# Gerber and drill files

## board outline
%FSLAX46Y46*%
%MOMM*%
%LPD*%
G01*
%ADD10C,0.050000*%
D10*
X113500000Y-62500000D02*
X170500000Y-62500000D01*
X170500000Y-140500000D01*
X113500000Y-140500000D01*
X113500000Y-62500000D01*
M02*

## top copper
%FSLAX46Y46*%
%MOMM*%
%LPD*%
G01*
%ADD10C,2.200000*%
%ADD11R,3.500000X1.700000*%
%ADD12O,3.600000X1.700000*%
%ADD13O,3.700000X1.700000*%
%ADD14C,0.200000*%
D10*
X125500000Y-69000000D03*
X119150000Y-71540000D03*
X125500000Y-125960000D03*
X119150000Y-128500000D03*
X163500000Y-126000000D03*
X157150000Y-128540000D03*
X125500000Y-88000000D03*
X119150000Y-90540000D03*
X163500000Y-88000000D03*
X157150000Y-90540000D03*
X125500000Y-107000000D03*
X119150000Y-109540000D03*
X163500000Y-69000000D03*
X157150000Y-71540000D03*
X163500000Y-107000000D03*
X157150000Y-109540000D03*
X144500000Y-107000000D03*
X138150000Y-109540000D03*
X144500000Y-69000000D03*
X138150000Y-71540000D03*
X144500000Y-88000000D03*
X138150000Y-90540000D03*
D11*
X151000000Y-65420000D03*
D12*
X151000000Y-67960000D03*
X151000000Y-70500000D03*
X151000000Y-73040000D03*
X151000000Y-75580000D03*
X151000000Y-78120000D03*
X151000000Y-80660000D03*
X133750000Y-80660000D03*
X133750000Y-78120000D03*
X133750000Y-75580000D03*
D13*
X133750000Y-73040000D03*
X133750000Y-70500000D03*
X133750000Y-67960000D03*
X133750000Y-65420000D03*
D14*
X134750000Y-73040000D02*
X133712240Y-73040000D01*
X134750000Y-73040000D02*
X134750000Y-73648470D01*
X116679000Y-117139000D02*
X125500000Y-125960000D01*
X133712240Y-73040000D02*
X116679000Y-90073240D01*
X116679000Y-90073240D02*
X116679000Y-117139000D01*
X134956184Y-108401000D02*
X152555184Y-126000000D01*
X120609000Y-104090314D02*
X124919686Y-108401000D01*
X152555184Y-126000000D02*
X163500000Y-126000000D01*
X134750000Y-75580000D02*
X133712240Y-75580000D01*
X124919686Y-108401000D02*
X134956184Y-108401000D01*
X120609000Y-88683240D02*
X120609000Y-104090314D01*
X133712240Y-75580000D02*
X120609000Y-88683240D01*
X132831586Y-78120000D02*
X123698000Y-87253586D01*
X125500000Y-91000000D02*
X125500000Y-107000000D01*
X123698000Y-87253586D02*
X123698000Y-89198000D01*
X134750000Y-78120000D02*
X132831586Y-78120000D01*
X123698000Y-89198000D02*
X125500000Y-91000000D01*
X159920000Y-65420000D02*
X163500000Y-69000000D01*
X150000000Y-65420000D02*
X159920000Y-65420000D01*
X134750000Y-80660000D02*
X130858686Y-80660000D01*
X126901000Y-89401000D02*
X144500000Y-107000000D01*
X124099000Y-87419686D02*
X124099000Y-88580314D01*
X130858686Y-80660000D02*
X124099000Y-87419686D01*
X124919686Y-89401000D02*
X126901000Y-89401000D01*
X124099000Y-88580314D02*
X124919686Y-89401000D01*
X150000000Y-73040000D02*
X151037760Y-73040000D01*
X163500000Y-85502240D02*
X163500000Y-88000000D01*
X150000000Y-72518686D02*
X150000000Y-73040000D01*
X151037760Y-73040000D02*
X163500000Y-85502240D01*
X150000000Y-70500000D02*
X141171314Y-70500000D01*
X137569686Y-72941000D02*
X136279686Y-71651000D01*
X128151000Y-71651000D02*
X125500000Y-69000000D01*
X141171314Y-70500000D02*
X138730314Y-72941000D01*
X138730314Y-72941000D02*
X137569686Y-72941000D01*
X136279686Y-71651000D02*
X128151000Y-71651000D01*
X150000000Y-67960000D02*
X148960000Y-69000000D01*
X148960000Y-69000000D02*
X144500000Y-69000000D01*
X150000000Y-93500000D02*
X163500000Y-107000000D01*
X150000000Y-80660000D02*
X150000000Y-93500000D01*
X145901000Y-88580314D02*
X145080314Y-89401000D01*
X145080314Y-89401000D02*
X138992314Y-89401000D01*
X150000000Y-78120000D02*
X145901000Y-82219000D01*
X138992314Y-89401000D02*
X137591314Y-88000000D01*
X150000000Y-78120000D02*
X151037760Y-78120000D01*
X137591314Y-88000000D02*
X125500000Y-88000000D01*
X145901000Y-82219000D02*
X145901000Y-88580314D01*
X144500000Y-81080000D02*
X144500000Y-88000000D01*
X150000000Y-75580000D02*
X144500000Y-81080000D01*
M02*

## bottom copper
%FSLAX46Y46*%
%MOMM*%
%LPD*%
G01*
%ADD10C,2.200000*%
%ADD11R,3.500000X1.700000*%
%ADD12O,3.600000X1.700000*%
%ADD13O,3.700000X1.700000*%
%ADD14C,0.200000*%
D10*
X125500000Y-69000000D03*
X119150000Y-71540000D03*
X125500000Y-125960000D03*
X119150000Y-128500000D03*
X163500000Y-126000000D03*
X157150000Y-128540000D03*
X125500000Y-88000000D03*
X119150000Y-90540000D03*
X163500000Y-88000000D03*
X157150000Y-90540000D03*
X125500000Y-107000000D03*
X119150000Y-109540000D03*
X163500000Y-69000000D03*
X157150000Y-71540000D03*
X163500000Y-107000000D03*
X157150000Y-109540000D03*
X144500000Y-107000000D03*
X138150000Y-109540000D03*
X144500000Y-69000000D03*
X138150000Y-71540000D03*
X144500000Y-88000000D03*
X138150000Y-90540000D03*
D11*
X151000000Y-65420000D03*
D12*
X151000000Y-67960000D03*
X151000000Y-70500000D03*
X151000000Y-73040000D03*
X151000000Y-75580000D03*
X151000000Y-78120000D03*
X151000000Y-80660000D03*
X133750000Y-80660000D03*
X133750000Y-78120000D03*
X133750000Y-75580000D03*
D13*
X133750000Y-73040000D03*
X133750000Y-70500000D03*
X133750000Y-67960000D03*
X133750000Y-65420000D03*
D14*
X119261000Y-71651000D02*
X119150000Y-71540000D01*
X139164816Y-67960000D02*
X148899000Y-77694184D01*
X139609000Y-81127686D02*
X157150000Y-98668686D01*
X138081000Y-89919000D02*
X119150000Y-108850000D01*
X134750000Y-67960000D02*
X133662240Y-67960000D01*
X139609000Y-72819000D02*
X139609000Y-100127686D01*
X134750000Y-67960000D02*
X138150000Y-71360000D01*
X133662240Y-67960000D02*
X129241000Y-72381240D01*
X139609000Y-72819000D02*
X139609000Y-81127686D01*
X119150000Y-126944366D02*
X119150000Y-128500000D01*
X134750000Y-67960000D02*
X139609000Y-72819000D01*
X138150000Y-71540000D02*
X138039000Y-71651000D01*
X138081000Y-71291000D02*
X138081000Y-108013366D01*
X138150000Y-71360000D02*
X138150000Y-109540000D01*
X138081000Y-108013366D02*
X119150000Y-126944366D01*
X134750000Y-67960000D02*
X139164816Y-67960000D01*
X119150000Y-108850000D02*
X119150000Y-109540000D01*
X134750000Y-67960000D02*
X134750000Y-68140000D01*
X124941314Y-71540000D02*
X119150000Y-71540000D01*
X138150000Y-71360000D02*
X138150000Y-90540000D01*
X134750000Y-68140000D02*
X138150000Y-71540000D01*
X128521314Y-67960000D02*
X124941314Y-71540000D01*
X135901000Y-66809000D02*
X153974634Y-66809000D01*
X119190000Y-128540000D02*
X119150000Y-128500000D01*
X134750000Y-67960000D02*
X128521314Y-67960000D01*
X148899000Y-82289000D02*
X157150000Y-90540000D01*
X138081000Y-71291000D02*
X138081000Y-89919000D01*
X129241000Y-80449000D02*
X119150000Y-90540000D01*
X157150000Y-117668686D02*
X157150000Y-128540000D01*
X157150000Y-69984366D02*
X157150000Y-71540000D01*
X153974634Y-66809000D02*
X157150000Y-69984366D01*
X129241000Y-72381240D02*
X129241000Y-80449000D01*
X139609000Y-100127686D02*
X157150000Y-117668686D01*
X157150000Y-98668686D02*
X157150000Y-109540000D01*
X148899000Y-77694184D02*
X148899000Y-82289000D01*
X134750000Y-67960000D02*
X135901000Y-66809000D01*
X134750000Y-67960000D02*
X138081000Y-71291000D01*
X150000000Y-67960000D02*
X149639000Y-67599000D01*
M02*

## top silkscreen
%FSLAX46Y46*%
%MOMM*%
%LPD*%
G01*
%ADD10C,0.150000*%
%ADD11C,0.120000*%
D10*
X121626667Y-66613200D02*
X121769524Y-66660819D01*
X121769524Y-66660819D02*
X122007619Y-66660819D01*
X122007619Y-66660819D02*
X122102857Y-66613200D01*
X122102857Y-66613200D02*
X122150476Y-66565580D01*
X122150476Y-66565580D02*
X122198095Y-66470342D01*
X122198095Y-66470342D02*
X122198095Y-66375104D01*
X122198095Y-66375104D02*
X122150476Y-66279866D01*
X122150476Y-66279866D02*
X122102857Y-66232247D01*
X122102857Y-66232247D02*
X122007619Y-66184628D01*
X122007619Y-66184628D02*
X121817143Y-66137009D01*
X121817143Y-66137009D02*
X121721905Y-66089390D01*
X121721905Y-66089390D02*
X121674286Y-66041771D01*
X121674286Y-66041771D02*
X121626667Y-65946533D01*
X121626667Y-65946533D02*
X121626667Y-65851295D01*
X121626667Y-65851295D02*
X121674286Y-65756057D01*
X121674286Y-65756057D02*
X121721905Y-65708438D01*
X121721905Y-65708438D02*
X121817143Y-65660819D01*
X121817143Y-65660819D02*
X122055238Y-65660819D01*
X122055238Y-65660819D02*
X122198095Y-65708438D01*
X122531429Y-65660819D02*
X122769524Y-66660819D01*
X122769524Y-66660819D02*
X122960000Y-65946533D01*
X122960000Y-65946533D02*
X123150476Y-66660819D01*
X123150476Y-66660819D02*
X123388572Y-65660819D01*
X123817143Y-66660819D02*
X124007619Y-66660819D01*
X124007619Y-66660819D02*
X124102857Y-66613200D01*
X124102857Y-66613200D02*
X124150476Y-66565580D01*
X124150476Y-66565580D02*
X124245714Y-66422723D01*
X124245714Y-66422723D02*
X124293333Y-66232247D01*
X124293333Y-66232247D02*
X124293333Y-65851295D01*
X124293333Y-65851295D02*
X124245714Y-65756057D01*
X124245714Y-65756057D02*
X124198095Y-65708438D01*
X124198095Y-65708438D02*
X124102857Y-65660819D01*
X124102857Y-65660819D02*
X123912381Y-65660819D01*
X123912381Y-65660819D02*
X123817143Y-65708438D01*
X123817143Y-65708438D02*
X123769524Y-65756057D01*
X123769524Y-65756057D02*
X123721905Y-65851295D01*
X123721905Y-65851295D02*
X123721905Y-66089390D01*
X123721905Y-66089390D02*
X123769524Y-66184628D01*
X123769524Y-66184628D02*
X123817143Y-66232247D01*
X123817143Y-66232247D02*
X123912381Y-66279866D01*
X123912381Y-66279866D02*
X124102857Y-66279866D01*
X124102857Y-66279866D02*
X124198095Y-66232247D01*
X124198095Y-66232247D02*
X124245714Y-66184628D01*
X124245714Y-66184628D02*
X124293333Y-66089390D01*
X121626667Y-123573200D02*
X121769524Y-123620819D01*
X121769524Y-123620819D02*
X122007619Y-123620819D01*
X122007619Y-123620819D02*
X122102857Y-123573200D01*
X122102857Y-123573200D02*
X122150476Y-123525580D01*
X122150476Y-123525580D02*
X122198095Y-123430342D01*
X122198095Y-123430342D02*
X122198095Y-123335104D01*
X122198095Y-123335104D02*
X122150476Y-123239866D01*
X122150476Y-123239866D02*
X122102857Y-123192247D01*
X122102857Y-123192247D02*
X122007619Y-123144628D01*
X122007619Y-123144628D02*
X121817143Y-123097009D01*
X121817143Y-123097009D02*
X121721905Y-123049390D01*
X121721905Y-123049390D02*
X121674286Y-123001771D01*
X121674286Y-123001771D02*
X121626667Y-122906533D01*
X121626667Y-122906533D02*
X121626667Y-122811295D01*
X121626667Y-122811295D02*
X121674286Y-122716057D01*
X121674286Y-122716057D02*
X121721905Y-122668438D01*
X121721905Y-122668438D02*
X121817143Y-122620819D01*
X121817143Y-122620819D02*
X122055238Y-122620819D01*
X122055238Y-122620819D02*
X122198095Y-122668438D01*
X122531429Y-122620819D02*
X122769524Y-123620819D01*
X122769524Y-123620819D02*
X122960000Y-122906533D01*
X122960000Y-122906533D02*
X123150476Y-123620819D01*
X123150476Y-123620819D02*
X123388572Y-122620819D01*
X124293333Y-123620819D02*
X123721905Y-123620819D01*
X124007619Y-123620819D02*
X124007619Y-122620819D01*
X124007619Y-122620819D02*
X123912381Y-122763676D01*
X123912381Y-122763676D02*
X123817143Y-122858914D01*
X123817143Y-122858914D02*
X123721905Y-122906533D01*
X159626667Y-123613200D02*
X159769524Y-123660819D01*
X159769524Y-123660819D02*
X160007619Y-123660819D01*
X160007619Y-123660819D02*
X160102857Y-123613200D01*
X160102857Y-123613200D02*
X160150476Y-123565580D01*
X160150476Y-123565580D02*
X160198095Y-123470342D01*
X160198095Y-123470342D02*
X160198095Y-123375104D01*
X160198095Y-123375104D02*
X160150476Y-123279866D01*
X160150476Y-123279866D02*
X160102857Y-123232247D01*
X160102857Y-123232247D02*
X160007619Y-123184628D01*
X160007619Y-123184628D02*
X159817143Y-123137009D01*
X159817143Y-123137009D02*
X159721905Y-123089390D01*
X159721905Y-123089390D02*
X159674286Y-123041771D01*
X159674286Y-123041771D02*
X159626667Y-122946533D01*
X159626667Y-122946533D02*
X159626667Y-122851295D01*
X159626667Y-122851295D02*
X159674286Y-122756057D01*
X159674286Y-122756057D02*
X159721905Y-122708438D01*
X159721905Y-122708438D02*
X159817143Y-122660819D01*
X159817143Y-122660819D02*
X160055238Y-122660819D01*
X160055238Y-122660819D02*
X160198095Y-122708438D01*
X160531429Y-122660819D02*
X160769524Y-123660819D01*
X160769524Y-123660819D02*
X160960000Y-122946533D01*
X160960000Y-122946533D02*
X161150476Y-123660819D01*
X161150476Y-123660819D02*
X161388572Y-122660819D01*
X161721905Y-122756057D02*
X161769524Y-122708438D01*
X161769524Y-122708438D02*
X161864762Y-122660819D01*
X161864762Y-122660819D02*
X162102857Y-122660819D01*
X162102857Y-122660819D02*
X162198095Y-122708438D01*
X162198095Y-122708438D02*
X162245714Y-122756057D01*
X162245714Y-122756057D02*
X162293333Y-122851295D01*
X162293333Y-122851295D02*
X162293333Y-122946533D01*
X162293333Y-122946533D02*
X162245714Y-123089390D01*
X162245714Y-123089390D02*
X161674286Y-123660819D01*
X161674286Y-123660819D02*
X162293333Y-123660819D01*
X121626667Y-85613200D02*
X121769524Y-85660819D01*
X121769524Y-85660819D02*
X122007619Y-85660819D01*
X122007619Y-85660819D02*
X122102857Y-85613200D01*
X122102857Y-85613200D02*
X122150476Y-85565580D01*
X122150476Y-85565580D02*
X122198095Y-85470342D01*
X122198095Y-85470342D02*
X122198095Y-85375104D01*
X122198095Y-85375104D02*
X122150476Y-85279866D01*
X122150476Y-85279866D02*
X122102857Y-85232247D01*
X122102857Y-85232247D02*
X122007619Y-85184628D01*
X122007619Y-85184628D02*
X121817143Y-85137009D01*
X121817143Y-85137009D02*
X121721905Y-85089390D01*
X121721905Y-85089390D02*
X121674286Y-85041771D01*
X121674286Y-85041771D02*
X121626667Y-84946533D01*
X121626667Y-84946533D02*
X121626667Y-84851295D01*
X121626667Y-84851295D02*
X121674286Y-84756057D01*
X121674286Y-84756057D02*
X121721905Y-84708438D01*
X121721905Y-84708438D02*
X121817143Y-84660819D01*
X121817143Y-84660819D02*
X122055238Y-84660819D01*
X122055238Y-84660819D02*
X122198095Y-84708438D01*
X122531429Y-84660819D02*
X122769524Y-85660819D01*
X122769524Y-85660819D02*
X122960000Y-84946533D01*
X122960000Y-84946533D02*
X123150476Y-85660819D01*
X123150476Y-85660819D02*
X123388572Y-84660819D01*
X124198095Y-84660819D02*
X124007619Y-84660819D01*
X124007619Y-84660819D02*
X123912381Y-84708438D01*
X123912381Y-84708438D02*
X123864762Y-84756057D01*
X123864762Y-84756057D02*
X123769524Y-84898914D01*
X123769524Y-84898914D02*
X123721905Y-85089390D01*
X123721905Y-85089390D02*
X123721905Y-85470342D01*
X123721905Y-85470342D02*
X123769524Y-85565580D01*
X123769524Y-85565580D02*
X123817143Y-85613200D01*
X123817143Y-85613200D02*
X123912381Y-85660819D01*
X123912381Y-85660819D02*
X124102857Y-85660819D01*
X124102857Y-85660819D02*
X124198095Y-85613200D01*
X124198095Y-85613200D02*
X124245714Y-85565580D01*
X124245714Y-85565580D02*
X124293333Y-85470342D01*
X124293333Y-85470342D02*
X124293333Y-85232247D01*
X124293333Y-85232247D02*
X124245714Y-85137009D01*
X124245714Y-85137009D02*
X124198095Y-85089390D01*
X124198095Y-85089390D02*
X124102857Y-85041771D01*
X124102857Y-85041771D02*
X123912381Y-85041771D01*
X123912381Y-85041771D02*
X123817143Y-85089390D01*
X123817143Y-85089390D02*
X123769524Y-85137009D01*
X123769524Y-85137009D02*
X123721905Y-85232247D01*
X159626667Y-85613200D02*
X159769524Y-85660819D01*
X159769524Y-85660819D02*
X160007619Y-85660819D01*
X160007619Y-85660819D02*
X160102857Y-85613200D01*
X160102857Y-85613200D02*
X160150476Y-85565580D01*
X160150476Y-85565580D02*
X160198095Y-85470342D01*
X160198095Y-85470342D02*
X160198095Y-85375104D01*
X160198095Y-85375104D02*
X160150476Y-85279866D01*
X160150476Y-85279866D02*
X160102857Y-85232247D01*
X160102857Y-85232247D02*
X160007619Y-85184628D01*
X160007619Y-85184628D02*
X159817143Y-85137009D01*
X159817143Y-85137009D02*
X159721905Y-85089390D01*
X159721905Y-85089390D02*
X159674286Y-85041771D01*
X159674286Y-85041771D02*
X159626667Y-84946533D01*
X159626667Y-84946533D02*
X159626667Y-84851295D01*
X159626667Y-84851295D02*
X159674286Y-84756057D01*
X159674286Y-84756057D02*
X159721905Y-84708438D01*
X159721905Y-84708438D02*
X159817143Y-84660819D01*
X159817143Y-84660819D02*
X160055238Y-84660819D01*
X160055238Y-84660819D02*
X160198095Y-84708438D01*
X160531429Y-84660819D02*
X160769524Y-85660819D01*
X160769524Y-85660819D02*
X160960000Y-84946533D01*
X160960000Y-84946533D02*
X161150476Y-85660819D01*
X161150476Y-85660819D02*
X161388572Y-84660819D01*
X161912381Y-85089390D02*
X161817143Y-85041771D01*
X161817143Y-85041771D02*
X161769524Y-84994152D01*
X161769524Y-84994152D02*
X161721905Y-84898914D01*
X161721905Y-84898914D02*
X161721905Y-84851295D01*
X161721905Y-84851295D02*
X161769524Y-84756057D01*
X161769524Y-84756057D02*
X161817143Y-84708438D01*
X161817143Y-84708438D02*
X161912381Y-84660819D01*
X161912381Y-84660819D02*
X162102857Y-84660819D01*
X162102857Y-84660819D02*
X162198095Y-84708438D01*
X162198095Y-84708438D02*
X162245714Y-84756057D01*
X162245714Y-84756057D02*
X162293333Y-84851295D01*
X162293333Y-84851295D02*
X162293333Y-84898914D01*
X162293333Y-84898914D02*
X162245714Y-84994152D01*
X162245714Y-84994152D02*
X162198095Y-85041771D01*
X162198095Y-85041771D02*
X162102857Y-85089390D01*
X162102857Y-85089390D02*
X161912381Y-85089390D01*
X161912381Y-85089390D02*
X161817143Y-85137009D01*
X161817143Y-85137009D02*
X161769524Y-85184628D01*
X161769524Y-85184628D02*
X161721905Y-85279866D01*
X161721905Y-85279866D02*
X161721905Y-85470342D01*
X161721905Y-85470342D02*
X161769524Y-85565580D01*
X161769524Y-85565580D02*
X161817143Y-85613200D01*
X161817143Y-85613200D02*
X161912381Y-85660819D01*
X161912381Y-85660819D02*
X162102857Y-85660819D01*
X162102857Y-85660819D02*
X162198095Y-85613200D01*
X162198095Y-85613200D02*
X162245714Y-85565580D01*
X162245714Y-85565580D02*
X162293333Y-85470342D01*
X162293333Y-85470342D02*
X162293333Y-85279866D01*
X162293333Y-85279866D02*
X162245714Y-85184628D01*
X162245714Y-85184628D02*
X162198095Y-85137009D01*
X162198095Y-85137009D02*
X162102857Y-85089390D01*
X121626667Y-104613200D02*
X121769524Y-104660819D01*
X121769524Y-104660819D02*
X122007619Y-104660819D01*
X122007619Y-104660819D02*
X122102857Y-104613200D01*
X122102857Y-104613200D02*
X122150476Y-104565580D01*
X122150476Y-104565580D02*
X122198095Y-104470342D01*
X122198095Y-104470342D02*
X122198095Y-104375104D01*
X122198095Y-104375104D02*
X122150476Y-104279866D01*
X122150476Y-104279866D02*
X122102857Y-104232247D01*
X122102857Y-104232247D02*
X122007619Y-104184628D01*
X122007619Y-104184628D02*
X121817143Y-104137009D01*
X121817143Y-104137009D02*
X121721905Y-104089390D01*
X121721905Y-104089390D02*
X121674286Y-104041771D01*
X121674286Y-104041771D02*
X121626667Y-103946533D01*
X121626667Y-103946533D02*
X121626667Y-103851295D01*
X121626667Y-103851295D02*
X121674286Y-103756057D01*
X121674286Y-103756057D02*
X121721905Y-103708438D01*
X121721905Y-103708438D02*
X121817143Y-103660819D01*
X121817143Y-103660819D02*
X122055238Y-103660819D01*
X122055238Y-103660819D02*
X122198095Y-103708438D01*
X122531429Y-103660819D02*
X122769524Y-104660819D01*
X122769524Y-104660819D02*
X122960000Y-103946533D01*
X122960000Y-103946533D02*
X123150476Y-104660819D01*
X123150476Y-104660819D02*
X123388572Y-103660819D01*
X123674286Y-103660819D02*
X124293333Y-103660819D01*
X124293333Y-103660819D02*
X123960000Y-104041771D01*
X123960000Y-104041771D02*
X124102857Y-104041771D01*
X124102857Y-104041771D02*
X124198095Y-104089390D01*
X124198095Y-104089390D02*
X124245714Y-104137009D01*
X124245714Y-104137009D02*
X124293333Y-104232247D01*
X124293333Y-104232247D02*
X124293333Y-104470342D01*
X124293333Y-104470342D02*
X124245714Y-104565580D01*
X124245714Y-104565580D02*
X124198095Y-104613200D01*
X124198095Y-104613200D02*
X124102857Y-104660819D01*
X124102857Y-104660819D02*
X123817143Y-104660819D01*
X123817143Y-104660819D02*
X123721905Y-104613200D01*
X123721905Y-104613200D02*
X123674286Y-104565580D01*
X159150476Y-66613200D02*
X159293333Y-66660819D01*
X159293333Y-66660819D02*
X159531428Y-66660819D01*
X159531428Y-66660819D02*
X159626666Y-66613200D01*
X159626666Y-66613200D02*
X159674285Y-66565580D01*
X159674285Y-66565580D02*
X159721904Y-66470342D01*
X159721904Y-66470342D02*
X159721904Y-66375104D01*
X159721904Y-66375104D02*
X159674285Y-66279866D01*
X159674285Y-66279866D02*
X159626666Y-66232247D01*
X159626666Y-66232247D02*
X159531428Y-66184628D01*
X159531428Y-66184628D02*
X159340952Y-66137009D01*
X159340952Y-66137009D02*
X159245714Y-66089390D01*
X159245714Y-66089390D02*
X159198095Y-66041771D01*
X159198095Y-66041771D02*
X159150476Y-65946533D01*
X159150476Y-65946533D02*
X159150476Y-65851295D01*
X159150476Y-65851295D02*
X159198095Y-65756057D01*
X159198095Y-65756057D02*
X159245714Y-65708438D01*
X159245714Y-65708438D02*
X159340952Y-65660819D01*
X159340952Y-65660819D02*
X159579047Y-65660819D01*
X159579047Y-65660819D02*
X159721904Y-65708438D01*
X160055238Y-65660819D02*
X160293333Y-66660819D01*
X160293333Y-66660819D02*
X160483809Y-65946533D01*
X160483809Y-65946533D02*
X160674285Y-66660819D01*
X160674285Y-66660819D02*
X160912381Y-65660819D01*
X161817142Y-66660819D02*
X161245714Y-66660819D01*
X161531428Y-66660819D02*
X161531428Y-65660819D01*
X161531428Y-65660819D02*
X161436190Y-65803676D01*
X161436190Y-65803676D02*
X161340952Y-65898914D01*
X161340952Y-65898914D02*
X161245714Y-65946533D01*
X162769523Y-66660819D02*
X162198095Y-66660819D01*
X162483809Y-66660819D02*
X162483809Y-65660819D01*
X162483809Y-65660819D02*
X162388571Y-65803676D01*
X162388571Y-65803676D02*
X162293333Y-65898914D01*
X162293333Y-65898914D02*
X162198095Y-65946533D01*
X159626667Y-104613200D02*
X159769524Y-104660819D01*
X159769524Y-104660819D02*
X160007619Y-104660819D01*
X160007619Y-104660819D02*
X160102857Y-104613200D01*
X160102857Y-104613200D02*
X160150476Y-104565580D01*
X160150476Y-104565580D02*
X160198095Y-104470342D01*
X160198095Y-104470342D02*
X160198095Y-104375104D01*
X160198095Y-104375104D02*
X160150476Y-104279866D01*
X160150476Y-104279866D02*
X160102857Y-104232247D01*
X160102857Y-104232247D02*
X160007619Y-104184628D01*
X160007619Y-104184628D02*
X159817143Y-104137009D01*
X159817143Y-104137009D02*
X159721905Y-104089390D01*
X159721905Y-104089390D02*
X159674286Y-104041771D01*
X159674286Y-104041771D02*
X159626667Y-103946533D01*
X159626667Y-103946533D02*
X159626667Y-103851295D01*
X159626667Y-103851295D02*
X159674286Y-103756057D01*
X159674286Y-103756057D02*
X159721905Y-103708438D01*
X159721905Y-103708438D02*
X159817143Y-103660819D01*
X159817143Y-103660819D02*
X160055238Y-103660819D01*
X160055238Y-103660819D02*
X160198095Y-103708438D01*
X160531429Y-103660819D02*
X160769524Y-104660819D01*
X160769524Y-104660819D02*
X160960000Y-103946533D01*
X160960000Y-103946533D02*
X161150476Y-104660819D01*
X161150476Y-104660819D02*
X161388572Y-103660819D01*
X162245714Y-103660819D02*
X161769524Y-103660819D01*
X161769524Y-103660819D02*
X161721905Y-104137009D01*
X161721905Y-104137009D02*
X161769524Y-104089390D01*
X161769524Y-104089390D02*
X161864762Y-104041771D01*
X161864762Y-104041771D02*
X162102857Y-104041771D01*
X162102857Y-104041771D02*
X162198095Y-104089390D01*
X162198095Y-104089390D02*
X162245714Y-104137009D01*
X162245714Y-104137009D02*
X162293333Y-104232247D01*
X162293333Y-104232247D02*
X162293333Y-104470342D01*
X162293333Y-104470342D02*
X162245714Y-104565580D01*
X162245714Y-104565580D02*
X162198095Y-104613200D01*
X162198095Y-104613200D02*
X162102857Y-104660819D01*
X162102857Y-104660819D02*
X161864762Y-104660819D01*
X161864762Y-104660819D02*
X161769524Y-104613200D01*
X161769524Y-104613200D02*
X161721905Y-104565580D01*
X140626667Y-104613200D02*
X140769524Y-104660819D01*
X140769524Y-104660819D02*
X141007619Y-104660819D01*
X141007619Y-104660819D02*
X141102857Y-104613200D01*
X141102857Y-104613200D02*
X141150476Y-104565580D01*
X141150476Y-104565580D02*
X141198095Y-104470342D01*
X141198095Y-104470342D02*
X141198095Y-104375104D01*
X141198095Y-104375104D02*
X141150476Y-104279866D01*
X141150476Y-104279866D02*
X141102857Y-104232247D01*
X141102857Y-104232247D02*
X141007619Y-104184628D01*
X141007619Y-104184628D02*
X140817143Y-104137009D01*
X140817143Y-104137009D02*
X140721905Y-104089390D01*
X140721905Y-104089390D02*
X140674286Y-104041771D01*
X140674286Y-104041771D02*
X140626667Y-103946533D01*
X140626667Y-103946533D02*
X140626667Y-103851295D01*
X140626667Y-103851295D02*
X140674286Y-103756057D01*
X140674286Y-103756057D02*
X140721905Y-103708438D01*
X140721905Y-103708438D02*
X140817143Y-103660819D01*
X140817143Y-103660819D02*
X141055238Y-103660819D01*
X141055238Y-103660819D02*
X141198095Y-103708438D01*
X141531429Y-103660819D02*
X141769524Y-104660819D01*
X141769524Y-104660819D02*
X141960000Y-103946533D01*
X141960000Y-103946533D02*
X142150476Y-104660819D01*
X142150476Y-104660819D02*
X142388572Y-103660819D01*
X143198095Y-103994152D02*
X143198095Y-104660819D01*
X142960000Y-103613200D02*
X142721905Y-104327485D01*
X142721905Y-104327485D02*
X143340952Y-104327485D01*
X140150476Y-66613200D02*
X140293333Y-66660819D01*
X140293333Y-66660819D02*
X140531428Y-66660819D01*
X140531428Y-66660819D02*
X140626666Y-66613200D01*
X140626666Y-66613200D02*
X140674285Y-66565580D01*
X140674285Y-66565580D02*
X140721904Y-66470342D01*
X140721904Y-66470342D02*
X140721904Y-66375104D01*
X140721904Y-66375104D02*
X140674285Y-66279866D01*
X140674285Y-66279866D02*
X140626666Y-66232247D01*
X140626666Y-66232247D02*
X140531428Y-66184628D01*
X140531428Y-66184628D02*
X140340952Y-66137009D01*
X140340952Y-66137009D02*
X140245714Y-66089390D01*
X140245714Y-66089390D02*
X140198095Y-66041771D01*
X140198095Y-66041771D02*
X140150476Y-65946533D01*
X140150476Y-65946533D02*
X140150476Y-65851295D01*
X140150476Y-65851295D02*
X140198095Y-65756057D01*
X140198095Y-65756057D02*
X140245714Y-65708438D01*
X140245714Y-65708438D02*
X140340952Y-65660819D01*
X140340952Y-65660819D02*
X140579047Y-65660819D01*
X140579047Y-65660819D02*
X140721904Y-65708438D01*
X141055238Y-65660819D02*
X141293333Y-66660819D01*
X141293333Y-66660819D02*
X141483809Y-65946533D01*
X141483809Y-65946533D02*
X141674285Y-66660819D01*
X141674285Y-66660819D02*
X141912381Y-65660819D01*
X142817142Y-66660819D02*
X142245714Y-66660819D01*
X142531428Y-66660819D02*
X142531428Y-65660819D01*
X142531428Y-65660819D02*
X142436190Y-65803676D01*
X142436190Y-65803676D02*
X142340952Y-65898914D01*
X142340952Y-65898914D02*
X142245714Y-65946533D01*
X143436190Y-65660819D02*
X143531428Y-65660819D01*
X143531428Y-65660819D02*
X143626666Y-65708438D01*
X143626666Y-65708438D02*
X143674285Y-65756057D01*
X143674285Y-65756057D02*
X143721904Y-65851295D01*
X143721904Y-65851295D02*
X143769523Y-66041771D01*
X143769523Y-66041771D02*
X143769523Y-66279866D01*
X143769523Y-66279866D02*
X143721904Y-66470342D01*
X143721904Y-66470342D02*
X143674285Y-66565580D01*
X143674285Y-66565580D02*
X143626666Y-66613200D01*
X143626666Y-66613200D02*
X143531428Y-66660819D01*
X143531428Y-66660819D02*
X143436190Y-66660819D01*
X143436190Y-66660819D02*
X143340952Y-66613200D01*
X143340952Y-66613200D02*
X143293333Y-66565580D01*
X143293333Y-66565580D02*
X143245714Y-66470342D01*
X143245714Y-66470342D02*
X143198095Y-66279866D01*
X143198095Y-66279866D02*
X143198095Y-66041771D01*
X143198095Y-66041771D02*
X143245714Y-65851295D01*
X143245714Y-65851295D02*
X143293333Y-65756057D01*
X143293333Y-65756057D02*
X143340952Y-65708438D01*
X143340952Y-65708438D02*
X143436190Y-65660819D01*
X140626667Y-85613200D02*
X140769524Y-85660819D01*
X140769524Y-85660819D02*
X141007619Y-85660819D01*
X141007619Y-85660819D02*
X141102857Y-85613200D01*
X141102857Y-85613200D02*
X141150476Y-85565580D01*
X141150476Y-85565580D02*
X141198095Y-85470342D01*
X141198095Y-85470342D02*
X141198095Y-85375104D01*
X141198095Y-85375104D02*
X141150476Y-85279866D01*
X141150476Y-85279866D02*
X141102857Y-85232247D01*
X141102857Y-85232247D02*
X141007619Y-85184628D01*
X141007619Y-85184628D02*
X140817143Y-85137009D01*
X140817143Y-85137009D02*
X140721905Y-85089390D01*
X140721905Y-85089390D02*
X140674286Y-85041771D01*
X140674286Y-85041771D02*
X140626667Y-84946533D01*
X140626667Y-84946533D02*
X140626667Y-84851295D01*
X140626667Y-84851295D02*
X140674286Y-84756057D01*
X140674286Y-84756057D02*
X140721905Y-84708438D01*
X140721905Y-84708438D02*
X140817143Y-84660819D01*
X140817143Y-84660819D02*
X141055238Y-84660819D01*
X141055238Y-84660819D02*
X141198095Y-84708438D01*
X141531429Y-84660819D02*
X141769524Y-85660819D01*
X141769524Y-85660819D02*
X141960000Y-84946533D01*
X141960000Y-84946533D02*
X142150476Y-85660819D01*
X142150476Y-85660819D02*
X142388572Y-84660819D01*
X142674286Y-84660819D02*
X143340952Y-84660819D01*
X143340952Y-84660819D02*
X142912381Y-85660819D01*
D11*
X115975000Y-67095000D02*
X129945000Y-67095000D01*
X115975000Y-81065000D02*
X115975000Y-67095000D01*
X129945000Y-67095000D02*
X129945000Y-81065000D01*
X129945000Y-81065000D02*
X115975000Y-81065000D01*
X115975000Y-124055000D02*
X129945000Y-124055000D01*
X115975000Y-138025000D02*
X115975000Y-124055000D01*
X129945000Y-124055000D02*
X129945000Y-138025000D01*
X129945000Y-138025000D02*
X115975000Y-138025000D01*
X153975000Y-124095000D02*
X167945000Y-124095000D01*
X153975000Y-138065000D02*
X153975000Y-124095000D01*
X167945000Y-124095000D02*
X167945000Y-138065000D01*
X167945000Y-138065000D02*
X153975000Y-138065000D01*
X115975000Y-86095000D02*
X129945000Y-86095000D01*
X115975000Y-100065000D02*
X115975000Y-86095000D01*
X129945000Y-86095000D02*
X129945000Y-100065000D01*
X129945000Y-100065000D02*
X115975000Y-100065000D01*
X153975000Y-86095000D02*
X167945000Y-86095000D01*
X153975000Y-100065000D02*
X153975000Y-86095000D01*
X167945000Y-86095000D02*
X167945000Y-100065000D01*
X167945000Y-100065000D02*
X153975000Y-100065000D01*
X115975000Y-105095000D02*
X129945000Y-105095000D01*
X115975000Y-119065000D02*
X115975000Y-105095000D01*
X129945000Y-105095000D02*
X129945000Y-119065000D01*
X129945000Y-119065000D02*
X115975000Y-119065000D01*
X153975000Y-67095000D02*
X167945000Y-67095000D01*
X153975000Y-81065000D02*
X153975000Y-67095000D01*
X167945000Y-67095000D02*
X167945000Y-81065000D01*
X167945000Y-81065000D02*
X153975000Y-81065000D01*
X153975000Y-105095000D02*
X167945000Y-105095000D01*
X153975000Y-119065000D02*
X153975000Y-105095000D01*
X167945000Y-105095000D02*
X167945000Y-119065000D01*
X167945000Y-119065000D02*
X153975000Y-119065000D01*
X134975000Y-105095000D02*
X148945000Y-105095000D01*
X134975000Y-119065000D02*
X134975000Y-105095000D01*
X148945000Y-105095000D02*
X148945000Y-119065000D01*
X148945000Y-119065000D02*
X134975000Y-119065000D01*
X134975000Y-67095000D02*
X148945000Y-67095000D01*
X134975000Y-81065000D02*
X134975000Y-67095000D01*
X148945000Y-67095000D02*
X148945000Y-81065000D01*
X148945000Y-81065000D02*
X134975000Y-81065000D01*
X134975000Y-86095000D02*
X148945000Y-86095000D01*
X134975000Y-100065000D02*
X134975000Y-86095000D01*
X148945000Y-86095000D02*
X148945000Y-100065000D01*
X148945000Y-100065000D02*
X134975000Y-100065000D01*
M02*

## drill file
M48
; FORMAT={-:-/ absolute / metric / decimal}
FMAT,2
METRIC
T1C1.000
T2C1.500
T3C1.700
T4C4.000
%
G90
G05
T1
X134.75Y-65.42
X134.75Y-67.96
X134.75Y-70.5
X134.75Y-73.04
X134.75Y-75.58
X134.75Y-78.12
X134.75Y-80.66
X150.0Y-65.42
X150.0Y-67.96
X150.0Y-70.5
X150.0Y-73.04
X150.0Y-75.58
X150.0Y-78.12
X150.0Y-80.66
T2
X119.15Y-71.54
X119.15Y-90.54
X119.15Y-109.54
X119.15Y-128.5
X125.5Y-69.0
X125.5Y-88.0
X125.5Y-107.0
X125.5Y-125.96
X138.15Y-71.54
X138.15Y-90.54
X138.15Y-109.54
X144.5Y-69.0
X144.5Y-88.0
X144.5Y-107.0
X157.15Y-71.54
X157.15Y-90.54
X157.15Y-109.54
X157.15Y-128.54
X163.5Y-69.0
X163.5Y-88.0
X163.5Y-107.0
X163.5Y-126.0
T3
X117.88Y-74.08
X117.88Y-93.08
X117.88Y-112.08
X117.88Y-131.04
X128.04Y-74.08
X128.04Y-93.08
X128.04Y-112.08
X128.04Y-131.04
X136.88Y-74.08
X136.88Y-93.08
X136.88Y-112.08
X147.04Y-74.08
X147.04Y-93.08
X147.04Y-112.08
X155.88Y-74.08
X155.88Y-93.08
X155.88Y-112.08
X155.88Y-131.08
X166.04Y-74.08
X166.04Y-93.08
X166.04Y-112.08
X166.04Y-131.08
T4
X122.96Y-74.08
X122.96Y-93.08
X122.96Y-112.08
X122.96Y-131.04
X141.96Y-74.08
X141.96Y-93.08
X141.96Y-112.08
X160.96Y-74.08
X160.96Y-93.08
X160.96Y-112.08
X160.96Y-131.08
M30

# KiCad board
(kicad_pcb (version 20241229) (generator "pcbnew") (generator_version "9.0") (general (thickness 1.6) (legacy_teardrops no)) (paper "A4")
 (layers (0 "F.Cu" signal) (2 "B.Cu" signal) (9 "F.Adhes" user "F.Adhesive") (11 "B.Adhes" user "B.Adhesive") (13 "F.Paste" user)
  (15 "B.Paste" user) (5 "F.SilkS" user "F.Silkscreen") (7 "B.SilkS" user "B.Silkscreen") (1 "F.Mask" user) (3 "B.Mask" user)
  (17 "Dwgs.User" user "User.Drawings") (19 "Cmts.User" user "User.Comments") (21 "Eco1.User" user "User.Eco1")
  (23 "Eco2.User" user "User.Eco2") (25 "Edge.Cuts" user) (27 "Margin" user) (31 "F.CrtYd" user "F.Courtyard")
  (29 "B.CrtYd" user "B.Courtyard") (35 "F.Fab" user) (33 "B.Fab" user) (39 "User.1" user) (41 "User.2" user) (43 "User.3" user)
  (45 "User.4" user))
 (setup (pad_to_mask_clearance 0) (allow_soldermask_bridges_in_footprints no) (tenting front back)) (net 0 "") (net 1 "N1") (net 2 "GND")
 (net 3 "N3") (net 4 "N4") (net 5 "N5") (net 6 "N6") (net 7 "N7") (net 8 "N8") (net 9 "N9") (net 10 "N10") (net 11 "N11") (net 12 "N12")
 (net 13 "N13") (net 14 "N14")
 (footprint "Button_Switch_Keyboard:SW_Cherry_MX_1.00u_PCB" (layer "F.Cu") (at 125.5 69)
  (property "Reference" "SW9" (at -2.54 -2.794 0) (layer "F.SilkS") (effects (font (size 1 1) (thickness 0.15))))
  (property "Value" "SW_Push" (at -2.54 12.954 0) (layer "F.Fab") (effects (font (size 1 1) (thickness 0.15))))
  (fp_line (start -9.525 -1.905) (end 4.445 -1.905) (stroke (width 0.12) (type solid)) (layer "F.SilkS"))
  (fp_line (start -9.525 12.065) (end -9.525 -1.905) (stroke (width 0.12) (type solid)) (layer "F.SilkS"))
  (fp_line (start 4.445 -1.905) (end 4.445 12.065) (stroke (width 0.12) (type solid)) (layer "F.SilkS"))
  (fp_line (start 4.445 12.065) (end -9.525 12.065) (stroke (width 0.12) (type solid)) (layer "F.SilkS"))
  (pad "" np_thru_hole circle (at -7.62 5.08) (size 1.7 1.7) (drill 1.7) (layers "*.Cu" "*.Mask"))
  (pad "" np_thru_hole circle (at -2.54 5.08) (size 4 4) (drill 4) (layers "*.Cu" "*.Mask"))
  (pad "" np_thru_hole circle (at 2.54 5.08) (size 1.7 1.7) (drill 1.7) (layers "*.Cu" "*.Mask"))
  (pad "1" thru_hole circle (at 0 0) (size 2.2 2.2) (drill 1.5) (layers "*.Cu" "*.Mask") (remove_unused_layers no) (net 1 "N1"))
  (pad "2" thru_hole circle (at -6.35 2.54) (size 2.2 2.2) (drill 1.5) (layers "*.Cu" "*.Mask") (remove_unused_layers no) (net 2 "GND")))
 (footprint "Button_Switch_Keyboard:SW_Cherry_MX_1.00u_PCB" (layer "F.Cu") (at 125.5 125.96)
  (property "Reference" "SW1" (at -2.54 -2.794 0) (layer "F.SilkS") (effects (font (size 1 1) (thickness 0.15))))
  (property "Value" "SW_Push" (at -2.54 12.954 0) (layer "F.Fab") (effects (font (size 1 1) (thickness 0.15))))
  (fp_line (start -9.525 -1.905) (end 4.445 -1.905) (stroke (width 0.12) (type solid)) (layer "F.SilkS"))
  (fp_line (start -9.525 12.065) (end -9.525 -1.905) (stroke (width 0.12) (type solid)) (layer "F.SilkS"))
  (fp_line (start 4.445 -1.905) (end 4.445 12.065) (stroke (width 0.12) (type solid)) (layer "F.SilkS"))
  (fp_line (start 4.445 12.065) (end -9.525 12.065) (stroke (width 0.12) (type solid)) (layer "F.SilkS"))
  (pad "" np_thru_hole circle (at -7.62 5.08) (size 1.7 1.7) (drill 1.7) (layers "*.Cu" "*.Mask"))
  (pad "" np_thru_hole circle (at -2.54 5.08) (size 4 4) (drill 4) (layers "*.Cu" "*.Mask"))
  (pad "" np_thru_hole circle (at 2.54 5.08) (size 1.7 1.7) (drill 1.7) (layers "*.Cu" "*.Mask"))
  (pad "1" thru_hole circle (at 0 0) (size 2.2 2.2) (drill 1.5) (layers "*.Cu" "*.Mask") (remove_unused_layers no) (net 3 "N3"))
  (pad "2" thru_hole circle (at -6.35 2.54) (size 2.2 2.2) (drill 1.5) (layers "*.Cu" "*.Mask") (remove_unused_layers no) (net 2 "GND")))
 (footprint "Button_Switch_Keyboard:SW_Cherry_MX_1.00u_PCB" (layer "F.Cu") (at 163.5 126)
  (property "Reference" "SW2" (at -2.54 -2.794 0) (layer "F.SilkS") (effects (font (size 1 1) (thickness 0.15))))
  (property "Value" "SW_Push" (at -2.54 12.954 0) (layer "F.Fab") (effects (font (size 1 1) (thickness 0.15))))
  (fp_line (start -9.525 -1.905) (end 4.445 -1.905) (stroke (width 0.12) (type solid)) (layer "F.SilkS"))
  (fp_line (start -9.525 12.065) (end -9.525 -1.905) (stroke (width 0.12) (type solid)) (layer "F.SilkS"))
  (fp_line (start 4.445 -1.905) (end 4.445 12.065) (stroke (width 0.12) (type solid)) (layer "F.SilkS"))
  (fp_line (start 4.445 12.065) (end -9.525 12.065) (stroke (width 0.12) (type solid)) (layer "F.SilkS"))
  (pad "" np_thru_hole circle (at -7.62 5.08) (size 1.7 1.7) (drill 1.7) (layers "*.Cu" "*.Mask"))
  (pad "" np_thru_hole circle (at -2.54 5.08) (size 4 4) (drill 4) (layers "*.Cu" "*.Mask"))
  (pad "" np_thru_hole circle (at 2.54 5.08) (size 1.7 1.7) (drill 1.7) (layers "*.Cu" "*.Mask"))
  (pad "1" thru_hole circle (at 0 0) (size 2.2 2.2) (drill 1.5) (layers "*.Cu" "*.Mask") (remove_unused_layers no) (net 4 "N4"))
  (pad "2" thru_hole circle (at -6.35 2.54) (size 2.2 2.2) (drill 1.5) (layers "*.Cu" "*.Mask") (remove_unused_layers no) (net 2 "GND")))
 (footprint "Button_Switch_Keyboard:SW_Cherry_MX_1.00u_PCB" (layer "F.Cu") (at 125.5 88)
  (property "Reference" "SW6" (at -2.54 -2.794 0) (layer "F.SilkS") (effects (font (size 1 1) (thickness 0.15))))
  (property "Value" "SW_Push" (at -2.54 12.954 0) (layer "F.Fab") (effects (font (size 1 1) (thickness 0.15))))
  (fp_line (start -9.525 -1.905) (end 4.445 -1.905) (stroke (width 0.12) (type solid)) (layer "F.SilkS"))
  (fp_line (start -9.525 12.065) (end -9.525 -1.905) (stroke (width 0.12) (type solid)) (layer "F.SilkS"))
  (fp_line (start 4.445 -1.905) (end 4.445 12.065) (stroke (width 0.12) (type solid)) (layer "F.SilkS"))
  (fp_line (start 4.445 12.065) (end -9.525 12.065) (stroke (width 0.12) (type solid)) (layer "F.SilkS"))
  (pad "" np_thru_hole circle (at -7.62 5.08) (size 1.7 1.7) (drill 1.7) (layers "*.Cu" "*.Mask"))
  (pad "" np_thru_hole circle (at -2.54 5.08) (size 4 4) (drill 4) (layers "*.Cu" "*.Mask"))
  (pad "" np_thru_hole circle (at 2.54 5.08) (size 1.7 1.7) (drill 1.7) (layers "*.Cu" "*.Mask"))
  (pad "1" thru_hole circle (at 0 0) (size 2.2 2.2) (drill 1.5) (layers "*.Cu" "*.Mask") (remove_unused_layers no) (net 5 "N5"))
  (pad "2" thru_hole circle (at -6.35 2.54) (size 2.2 2.2) (drill 1.5) (layers "*.Cu" "*.Mask") (remove_unused_layers no) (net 2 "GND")))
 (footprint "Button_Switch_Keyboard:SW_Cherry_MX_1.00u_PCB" (layer "F.Cu") (at 163.5 88)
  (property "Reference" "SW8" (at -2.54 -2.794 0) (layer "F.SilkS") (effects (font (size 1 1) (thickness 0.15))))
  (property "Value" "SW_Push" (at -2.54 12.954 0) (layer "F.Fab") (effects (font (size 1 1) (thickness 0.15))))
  (fp_line (start -9.525 -1.905) (end 4.445 -1.905) (stroke (width 0.12) (type solid)) (layer "F.SilkS"))
  (fp_line (start -9.525 12.065) (end -9.525 -1.905) (stroke (width 0.12) (type solid)) (layer "F.SilkS"))
  (fp_line (start 4.445 -1.905) (end 4.445 12.065) (stroke (width 0.12) (type solid)) (layer "F.SilkS"))
  (fp_line (start 4.445 12.065) (end -9.525 12.065) (stroke (width 0.12) (type solid)) (layer "F.SilkS"))
  (pad "" np_thru_hole circle (at -7.62 5.08) (size 1.7 1.7) (drill 1.7) (layers "*.Cu" "*.Mask"))
  (pad "" np_thru_hole circle (at -2.54 5.08) (size 4 4) (drill 4) (layers "*.Cu" "*.Mask"))
  (pad "" np_thru_hole circle (at 2.54 5.08) (size 1.7 1.7) (drill 1.7) (layers "*.Cu" "*.Mask"))
  (pad "1" thru_hole circle (at 0 0) (size 2.2 2.2) (drill 1.5) (layers "*.Cu" "*.Mask") (remove_unused_layers no) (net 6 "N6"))
  (pad "2" thru_hole circle (at -6.35 2.54) (size 2.2 2.2) (drill 1.5) (layers "*.Cu" "*.Mask") (remove_unused_layers no) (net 2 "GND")))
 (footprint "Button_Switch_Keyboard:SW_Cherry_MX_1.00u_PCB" (layer "F.Cu") (at 125.5 107)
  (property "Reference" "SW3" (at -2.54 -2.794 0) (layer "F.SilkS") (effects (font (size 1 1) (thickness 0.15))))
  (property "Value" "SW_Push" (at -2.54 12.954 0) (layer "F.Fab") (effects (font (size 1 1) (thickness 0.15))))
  (fp_line (start -9.525 -1.905) (end 4.445 -1.905) (stroke (width 0.12) (type solid)) (layer "F.SilkS"))
  (fp_line (start -9.525 12.065) (end -9.525 -1.905) (stroke (width 0.12) (type solid)) (layer "F.SilkS"))
  (fp_line (start 4.445 -1.905) (end 4.445 12.065) (stroke (width 0.12) (type solid)) (layer "F.SilkS"))
  (fp_line (start 4.445 12.065) (end -9.525 12.065) (stroke (width 0.12) (type solid)) (layer "F.SilkS"))
  (pad "" np_thru_hole circle (at -7.62 5.08) (size 1.7 1.7) (drill 1.7) (layers "*.Cu" "*.Mask"))
  (pad "" np_thru_hole circle (at -2.54 5.08) (size 4 4) (drill 4) (layers "*.Cu" "*.Mask"))
  (pad "" np_thru_hole circle (at 2.54 5.08) (size 1.7 1.7) (drill 1.7) (layers "*.Cu" "*.Mask"))
  (pad "1" thru_hole circle (at 0 0) (size 2.2 2.2) (drill 1.5) (layers "*.Cu" "*.Mask") (remove_unused_layers no) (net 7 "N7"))
  (pad "2" thru_hole circle (at -6.35 2.54) (size 2.2 2.2) (drill 1.5) (layers "*.Cu" "*.Mask") (remove_unused_layers no) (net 2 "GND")))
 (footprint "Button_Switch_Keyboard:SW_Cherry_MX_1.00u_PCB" (layer "F.Cu") (at 163.5 69)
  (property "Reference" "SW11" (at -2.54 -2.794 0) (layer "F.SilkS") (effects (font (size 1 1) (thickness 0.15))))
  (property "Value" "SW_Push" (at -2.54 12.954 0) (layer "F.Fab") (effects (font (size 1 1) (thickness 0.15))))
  (fp_line (start -9.525 -1.905) (end 4.445 -1.905) (stroke (width 0.12) (type solid)) (layer "F.SilkS"))
  (fp_line (start -9.525 12.065) (end -9.525 -1.905) (stroke (width 0.12) (type solid)) (layer "F.SilkS"))
  (fp_line (start 4.445 -1.905) (end 4.445 12.065) (stroke (width 0.12) (type solid)) (layer "F.SilkS"))
  (fp_line (start 4.445 12.065) (end -9.525 12.065) (stroke (width 0.12) (type solid)) (layer "F.SilkS"))
  (pad "" np_thru_hole circle (at -7.62 5.08) (size 1.7 1.7) (drill 1.7) (layers "*.Cu" "*.Mask"))
  (pad "" np_thru_hole circle (at -2.54 5.08) (size 4 4) (drill 4) (layers "*.Cu" "*.Mask"))
  (pad "" np_thru_hole circle (at 2.54 5.08) (size 1.7 1.7) (drill 1.7) (layers "*.Cu" "*.Mask"))
  (pad "1" thru_hole circle (at 0 0) (size 2.2 2.2) (drill 1.5) (layers "*.Cu" "*.Mask") (remove_unused_layers no) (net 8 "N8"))
  (pad "2" thru_hole circle (at -6.35 2.54) (size 2.2 2.2) (drill 1.5) (layers "*.Cu" "*.Mask") (remove_unused_layers no) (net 2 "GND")))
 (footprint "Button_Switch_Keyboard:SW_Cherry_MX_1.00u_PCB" (layer "F.Cu") (at 163.5 107)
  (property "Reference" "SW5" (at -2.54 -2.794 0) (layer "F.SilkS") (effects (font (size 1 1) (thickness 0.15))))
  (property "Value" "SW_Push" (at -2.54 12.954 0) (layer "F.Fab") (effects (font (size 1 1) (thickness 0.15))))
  (fp_line (start -9.525 -1.905) (end 4.445 -1.905) (stroke (width 0.12) (type solid)) (layer "F.SilkS"))
  (fp_line (start -9.525 12.065) (end -9.525 -1.905) (stroke (width 0.12) (type solid)) (layer "F.SilkS"))
  (fp_line (start 4.445 -1.905) (end 4.445 12.065) (stroke (width 0.12) (type solid)) (layer "F.SilkS"))
  (fp_line (start 4.445 12.065) (end -9.525 12.065) (stroke (width 0.12) (type solid)) (layer "F.SilkS"))
  (pad "" np_thru_hole circle (at -7.62 5.08) (size 1.7 1.7) (drill 1.7) (layers "*.Cu" "*.Mask"))
  (pad "" np_thru_hole circle (at -2.54 5.08) (size 4 4) (drill 4) (layers "*.Cu" "*.Mask"))
  (pad "" np_thru_hole circle (at 2.54 5.08) (size 1.7 1.7) (drill 1.7) (layers "*.Cu" "*.Mask"))
  (pad "1" thru_hole circle (at 0 0) (size 2.2 2.2) (drill 1.5) (layers "*.Cu" "*.Mask") (remove_unused_layers no) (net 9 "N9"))
  (pad "2" thru_hole circle (at -6.35 2.54) (size 2.2 2.2) (drill 1.5) (layers "*.Cu" "*.Mask") (remove_unused_layers no) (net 2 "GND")))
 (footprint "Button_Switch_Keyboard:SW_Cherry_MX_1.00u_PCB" (layer "F.Cu") (at 144.5 107)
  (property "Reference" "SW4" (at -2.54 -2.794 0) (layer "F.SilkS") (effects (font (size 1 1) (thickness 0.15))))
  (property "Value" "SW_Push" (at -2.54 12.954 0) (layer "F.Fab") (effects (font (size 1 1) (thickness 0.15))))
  (fp_line (start -9.525 -1.905) (end 4.445 -1.905) (stroke (width 0.12) (type solid)) (layer "F.SilkS"))
  (fp_line (start -9.525 12.065) (end -9.525 -1.905) (stroke (width 0.12) (type solid)) (layer "F.SilkS"))
  (fp_line (start 4.445 -1.905) (end 4.445 12.065) (stroke (width 0.12) (type solid)) (layer "F.SilkS"))
  (fp_line (start 4.445 12.065) (end -9.525 12.065) (stroke (width 0.12) (type solid)) (layer "F.SilkS"))
  (pad "" np_thru_hole circle (at -7.62 5.08) (size 1.7 1.7) (drill 1.7) (layers "*.Cu" "*.Mask"))
  (pad "" np_thru_hole circle (at -2.54 5.08) (size 4 4) (drill 4) (layers "*.Cu" "*.Mask"))
  (pad "" np_thru_hole circle (at 2.54 5.08) (size 1.7 1.7) (drill 1.7) (layers "*.Cu" "*.Mask"))
  (pad "1" thru_hole circle (at 0 0) (size 2.2 2.2) (drill 1.5) (layers "*.Cu" "*.Mask") (remove_unused_layers no) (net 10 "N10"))
  (pad "2" thru_hole circle (at -6.35 2.54) (size 2.2 2.2) (drill 1.5) (layers "*.Cu" "*.Mask") (remove_unused_layers no) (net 2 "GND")))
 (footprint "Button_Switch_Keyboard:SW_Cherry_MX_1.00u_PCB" (layer "F.Cu") (at 144.5 69)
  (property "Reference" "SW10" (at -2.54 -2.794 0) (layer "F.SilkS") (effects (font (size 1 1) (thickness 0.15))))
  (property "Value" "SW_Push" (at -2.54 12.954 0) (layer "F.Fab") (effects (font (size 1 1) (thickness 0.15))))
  (fp_line (start -9.525 -1.905) (end 4.445 -1.905) (stroke (width 0.12) (type solid)) (layer "F.SilkS"))
  (fp_line (start -9.525 12.065) (end -9.525 -1.905) (stroke (width 0.12) (type solid)) (layer "F.SilkS"))
  (fp_line (start 4.445 -1.905) (end 4.445 12.065) (stroke (width 0.12) (type solid)) (layer "F.SilkS"))
  (fp_line (start 4.445 12.065) (end -9.525 12.065) (stroke (width 0.12) (type solid)) (layer "F.SilkS"))
  (pad "" np_thru_hole circle (at -7.62 5.08) (size 1.7 1.7) (drill 1.7) (layers "*.Cu" "*.Mask"))
  (pad "" np_thru_hole circle (at -2.54 5.08) (size 4 4) (drill 4) (layers "*.Cu" "*.Mask"))
  (pad "" np_thru_hole circle (at 2.54 5.08) (size 1.7 1.7) (drill 1.7) (layers "*.Cu" "*.Mask"))
  (pad "1" thru_hole circle (at 0 0) (size 2.2 2.2) (drill 1.5) (layers "*.Cu" "*.Mask") (remove_unused_layers no) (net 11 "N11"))
  (pad "2" thru_hole circle (at -6.35 2.54) (size 2.2 2.2) (drill 1.5) (layers "*.Cu" "*.Mask") (remove_unused_layers no) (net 2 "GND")))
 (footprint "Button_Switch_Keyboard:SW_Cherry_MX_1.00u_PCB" (layer "F.Cu") (at 144.5 88)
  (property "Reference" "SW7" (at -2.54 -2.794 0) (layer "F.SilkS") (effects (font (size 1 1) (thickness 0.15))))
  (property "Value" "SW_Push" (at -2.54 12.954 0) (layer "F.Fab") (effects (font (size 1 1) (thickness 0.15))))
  (fp_line (start -9.525 -1.905) (end 4.445 -1.905) (stroke (width 0.12) (type solid)) (layer "F.SilkS"))
  (fp_line (start -9.525 12.065) (end -9.525 -1.905) (stroke (width 0.12) (type solid)) (layer "F.SilkS"))
  (fp_line (start 4.445 -1.905) (end 4.445 12.065) (stroke (width 0.12) (type solid)) (layer "F.SilkS"))
  (fp_line (start 4.445 12.065) (end -9.525 12.065) (stroke (width 0.12) (type solid)) (layer "F.SilkS"))
  (pad "" np_thru_hole circle (at -7.62 5.08) (size 1.7 1.7) (drill 1.7) (layers "*.Cu" "*.Mask"))
  (pad "" np_thru_hole circle (at -2.54 5.08) (size 4 4) (drill 4) (layers "*.Cu" "*.Mask"))
  (pad "" np_thru_hole circle (at 2.54 5.08) (size 1.7 1.7) (drill 1.7) (layers "*.Cu" "*.Mask"))
  (pad "1" thru_hole circle (at 0 0) (size 2.2 2.2) (drill 1.5) (layers "*.Cu" "*.Mask") (remove_unused_layers no) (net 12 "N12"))
  (pad "2" thru_hole circle (at -6.35 2.54) (size 2.2 2.2) (drill 1.5) (layers "*.Cu" "*.Mask") (remove_unused_layers no) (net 2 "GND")))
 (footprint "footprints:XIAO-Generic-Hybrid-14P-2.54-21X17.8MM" (layer "B.Cu") (at 142.375 73.04 180)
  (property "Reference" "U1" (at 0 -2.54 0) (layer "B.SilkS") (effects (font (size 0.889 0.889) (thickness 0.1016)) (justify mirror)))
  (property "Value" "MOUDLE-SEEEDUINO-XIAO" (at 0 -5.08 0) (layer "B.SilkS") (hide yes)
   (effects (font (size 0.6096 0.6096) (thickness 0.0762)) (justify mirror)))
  (pad "1" thru_hole rect (at -7.625 7.62 180) (size 3.5 1.7) (drill 1 (offset -1 0)) (layers "*.Cu" "*.Mask") (remove_unused_layers no)
   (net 8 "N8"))
  (pad "2" thru_hole oval (at -7.625 5.08 180) (size 3.6 1.7) (drill 1 (offset -1 0)) (layers "*.Cu" "*.Mask") (remove_unused_layers no)
   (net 11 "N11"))
  (pad "3" thru_hole oval (at -7.625 2.54 180) (size 3.6 1.7) (drill 1 (offset -1 0)) (layers "*.Cu" "*.Mask") (remove_unused_layers no)
   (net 1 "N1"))
  (pad "4" thru_hole oval (at -7.625 0 180) (size 3.6 1.7) (drill 1 (offset -1 0)) (layers "*.Cu" "*.Mask") (remove_unused_layers no)
   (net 6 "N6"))
  (pad "5" thru_hole oval (at -7.625 -2.54 180) (size 3.6 1.7) (drill 1 (offset -1 0)) (layers "*.Cu" "*.Mask") (remove_unused_layers no)
   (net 12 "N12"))
  (pad "6" thru_hole oval (at -7.625 -5.08) (size 3.6 1.7) (drill 1 (offset 1 0)) (layers "*.Cu" "*.Mask") (remove_unused_layers no)
   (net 5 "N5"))
  (pad "7" thru_hole oval (at -7.625 -7.62 180) (size 3.6 1.7) (drill 1 (offset -1 0)) (layers "*.Cu" "*.Mask") (remove_unused_layers no)
   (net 9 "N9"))
  (pad "8" thru_hole oval (at 7.625 -7.62 180) (size 3.6 1.7) (drill 1 (offset 1 0)) (layers "*.Cu" "*.Mask") (remove_unused_layers no)
   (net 10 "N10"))
  (pad "9" thru_hole oval (at 7.625 -5.08 180) (size 3.6 1.7) (drill 1 (offset 1 0)) (layers "*.Cu" "*.Mask") (remove_unused_layers no)
   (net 7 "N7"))
  (pad "10" thru_hole oval (at 7.625 -2.54 180) (size 3.6 1.7) (drill 1 (offset 1 0)) (layers "*.Cu" "*.Mask") (remove_unused_layers no)
   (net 4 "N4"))
  (pad "11" thru_hole oval (at 7.625 0 180) (size 3.7 1.7) (drill 1 (offset 1 0)) (layers "*.Cu" "*.Mask") (remove_unused_layers no)
   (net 3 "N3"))
  (pad "12" thru_hole oval (at 7.625 2.54 180) (size 3.7 1.7) (drill 1 (offset 1 0)) (layers "*.Cu" "*.Mask") (remove_unused_layers no)
   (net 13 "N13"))
  (pad "13" thru_hole oval (at 7.625 5.08 180) (size 3.7 1.7) (drill 1 (offset 1 0)) (layers "*.Cu" "*.Mask") (remove_unused_layers no)
   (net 2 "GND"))
  (pad "14" thru_hole oval (at 7.625 7.62 180) (size 3.7 1.7) (drill 1 (offset 1 0)) (layers "*.Cu" "*.Mask") (remove_unused_layers no)
   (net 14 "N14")))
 (gr_rect (start 113.5 62.5) (end 170.5 140.5) (stroke (width 0.05) (type default)) (fill no) (layer "Edge.Cuts"))
 (segment (start 119.261 71.651) (end 119.15 71.54) (width 0.2) (layer "B.Cu") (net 2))
 (segment (start 139.164816 67.96) (end 148.899 77.694184) (width 0.2) (layer "B.Cu") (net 2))
 (segment (start 139.609 81.127686) (end 157.15 98.668686) (width 0.2) (layer "B.Cu") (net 2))
 (segment (start 138.081 89.919) (end 119.15 108.85) (width 0.2) (layer "B.Cu") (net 2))
 (segment (start 134.75 67.96) (end 133.66224 67.96) (width 0.2) (layer "B.Cu") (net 2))
 (segment (start 139.609 72.819) (end 139.609 100.127686) (width 0.2) (layer "B.Cu") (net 2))
 (segment (start 134.75 67.96) (end 138.15 71.36) (width 0.2) (layer "B.Cu") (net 2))
 (segment (start 133.66224 67.96) (end 129.241 72.38124) (width 0.2) (layer "B.Cu") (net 2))
 (segment (start 139.609 72.819) (end 139.609 81.127686) (width 0.2) (layer "B.Cu") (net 2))
 (segment (start 119.15 126.944366) (end 119.15 128.5) (width 0.2) (layer "B.Cu") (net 2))
 (segment (start 134.75 67.96) (end 139.609 72.819) (width 0.2) (layer "B.Cu") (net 2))
 (segment (start 138.15 71.54) (end 138.039 71.651) (width 0.2) (layer "B.Cu") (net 2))
 (segment (start 138.081 71.291) (end 138.081 108.013366) (width 0.2) (layer "B.Cu") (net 2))
 (segment (start 138.15 71.36) (end 138.15 109.54) (width 0.2) (layer "B.Cu") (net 2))
 (segment (start 138.081 108.013366) (end 119.15 126.944366) (width 0.2) (layer "B.Cu") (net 2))
 (segment (start 134.75 67.96) (end 139.164816 67.96) (width 0.2) (layer "B.Cu") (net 2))
 (segment (start 119.15 108.85) (end 119.15 109.54) (width 0.2) (layer "B.Cu") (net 2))
 (segment (start 134.75 67.96) (end 134.75 68.14) (width 0.2) (layer "B.Cu") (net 2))
 (segment (start 124.941314 71.54) (end 119.15 71.54) (width 0.2) (layer "B.Cu") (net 2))
 (segment (start 138.15 71.36) (end 138.15 90.54) (width 0.2) (layer "B.Cu") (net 2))
 (segment (start 134.75 68.14) (end 138.15 71.54) (width 0.2) (layer "B.Cu") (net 2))
 (segment (start 128.521314 67.96) (end 124.941314 71.54) (width 0.2) (layer "B.Cu") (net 2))
 (segment (start 135.901 66.809) (end 153.974634 66.809) (width 0.2) (layer "B.Cu") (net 2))
 (segment (start 119.19 128.54) (end 119.15 128.5) (width 0.2) (layer "B.Cu") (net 2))
 (segment (start 134.75 67.96) (end 128.521314 67.96) (width 0.2) (layer "B.Cu") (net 2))
 (segment (start 148.899 82.289) (end 157.15 90.54) (width 0.2) (layer "B.Cu") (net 2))
 (segment (start 138.081 71.291) (end 138.081 89.919) (width 0.2) (layer "B.Cu") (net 2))
 (segment (start 129.241 80.449) (end 119.15 90.54) (width 0.2) (layer "B.Cu") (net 2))
 (segment (start 157.15 117.668686) (end 157.15 128.54) (width 0.2) (layer "B.Cu") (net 2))
 (segment (start 157.15 69.984366) (end 157.15 71.54) (width 0.2) (layer "B.Cu") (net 2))
 (segment (start 153.974634 66.809) (end 157.15 69.984366) (width 0.2) (layer "B.Cu") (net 2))
 (segment (start 129.241 72.38124) (end 129.241 80.449) (width 0.2) (layer "B.Cu") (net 2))
 (segment (start 139.609 100.127686) (end 157.15 117.668686) (width 0.2) (layer "B.Cu") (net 2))
 (segment (start 157.15 98.668686) (end 157.15 109.54) (width 0.2) (layer "B.Cu") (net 2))
 (segment (start 148.899 77.694184) (end 148.899 82.289) (width 0.2) (layer "B.Cu") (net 2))
 (segment (start 134.75 67.96) (end 135.901 66.809) (width 0.2) (layer "B.Cu") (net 2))
 (segment (start 134.75 67.96) (end 138.081 71.291) (width 0.2) (layer "B.Cu") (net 2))
 (segment (start 134.75 73.04) (end 133.71224 73.04) (width 0.2) (layer "F.Cu") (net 3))
 (segment (start 134.75 73.04) (end 134.75 73.64847) (width 0.2) (layer "F.Cu") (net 3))
 (segment (start 116.679 117.139) (end 125.5 125.96) (width 0.2) (layer "F.Cu") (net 3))
 (segment (start 133.71224 73.04) (end 116.679 90.07324) (width 0.2) (layer "F.Cu") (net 3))
 (segment (start 116.679 90.07324) (end 116.679 117.139) (width 0.2) (layer "F.Cu") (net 3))
 (segment (start 134.956184 108.401) (end 152.555184 126) (width 0.2) (layer "F.Cu") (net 4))
 (segment (start 120.609 104.090314) (end 124.919686 108.401) (width 0.2) (layer "F.Cu") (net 4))
 (segment (start 152.555184 126) (end 163.5 126) (width 0.2) (layer "F.Cu") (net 4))
 (segment (start 134.75 75.58) (end 133.71224 75.58) (width 0.2) (layer "F.Cu") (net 4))
 (segment (start 124.919686 108.401) (end 134.956184 108.401) (width 0.2) (layer "F.Cu") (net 4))
 (segment (start 120.609 88.68324) (end 120.609 104.090314) (width 0.2) (layer "F.Cu") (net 4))
 (segment (start 133.71224 75.58) (end 120.609 88.68324) (width 0.2) (layer "F.Cu") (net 4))
 (segment (start 132.831586 78.12) (end 123.698 87.253586) (width 0.2) (layer "F.Cu") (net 7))
 (segment (start 125.5 91) (end 125.5 107) (width 0.2) (layer "F.Cu") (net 7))
 (segment (start 123.698 87.253586) (end 123.698 89.198) (width 0.2) (layer "F.Cu") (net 7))
 (segment (start 134.75 78.12) (end 132.831586 78.12) (width 0.2) (layer "F.Cu") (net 7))
 (segment (start 123.698 89.198) (end 125.5 91) (width 0.2) (layer "F.Cu") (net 7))
 (segment (start 159.92 65.42) (end 163.5 69) (width 0.2) (layer "F.Cu") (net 8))
 (segment (start 150 65.42) (end 159.92 65.42) (width 0.2) (layer "F.Cu") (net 8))
 (segment (start 134.75 80.66) (end 130.858686 80.66) (width 0.2) (layer "F.Cu") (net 10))
 (segment (start 126.901 89.401) (end 144.5 107) (width 0.2) (layer "F.Cu") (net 10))
 (segment (start 124.099 87.419686) (end 124.099 88.580314) (width 0.2) (layer "F.Cu") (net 10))
 (segment (start 130.858686 80.66) (end 124.099 87.419686) (width 0.2) (layer "F.Cu") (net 10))
 (segment (start 124.919686 89.401) (end 126.901 89.401) (width 0.2) (layer "F.Cu") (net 10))
 (segment (start 124.099 88.580314) (end 124.919686 89.401) (width 0.2) (layer "F.Cu") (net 10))
 (segment (start 150 73.04) (end 151.03776 73.04) (width 0.2) (layer "F.Cu") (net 6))
 (segment (start 163.5 85.50224) (end 163.5 88) (width 0.2) (layer "F.Cu") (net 6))
 (segment (start 150 72.518686) (end 150 73.04) (width 0.2) (layer "F.Cu") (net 6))
 (segment (start 151.03776 73.04) (end 163.5 85.50224) (width 0.2) (layer "F.Cu") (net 6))
 (segment (start 150 70.5) (end 141.171314 70.5) (width 0.2) (layer "F.Cu") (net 1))
 (segment (start 137.569686 72.941) (end 136.279686 71.651) (width 0.2) (layer "F.Cu") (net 1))
 (segment (start 128.151 71.651) (end 125.5 69) (width 0.2) (layer "F.Cu") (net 1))
 (segment (start 141.171314 70.5) (end 138.730314 72.941) (width 0.2) (layer "F.Cu") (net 1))
 (segment (start 138.730314 72.941) (end 137.569686 72.941) (width 0.2) (layer "F.Cu") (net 1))
 (segment (start 136.279686 71.651) (end 128.151 71.651) (width 0.2) (layer "F.Cu") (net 1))
 (segment (start 150 67.96) (end 148.96 69) (width 0.2) (layer "F.Cu") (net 11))
 (segment (start 148.96 69) (end 144.5 69) (width 0.2) (layer "F.Cu") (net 11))
 (segment (start 150 67.96) (end 149.639 67.599) (width 0.2) (layer "B.Cu") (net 11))
 (segment (start 150 93.5) (end 163.5 107) (width 0.2) (layer "F.Cu") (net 9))
 (segment (start 150 80.66) (end 150 93.5) (width 0.2) (layer "F.Cu") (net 9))
 (segment (start 145.901 88.580314) (end 145.080314 89.401) (width 0.2) (layer "F.Cu") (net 5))
 (segment (start 145.080314 89.401) (end 138.992314 89.401) (width 0.2) (layer "F.Cu") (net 5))
 (segment (start 150 78.12) (end 145.901 82.219) (width 0.2) (layer "F.Cu") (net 5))
 (segment (start 138.992314 89.401) (end 137.591314 88) (width 0.2) (layer "F.Cu") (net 5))
 (segment (start 150 78.12) (end 151.03776 78.12) (width 0.2) (layer "F.Cu") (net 5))
 (segment (start 137.591314 88) (end 125.5 88) (width 0.2) (layer "F.Cu") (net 5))
 (segment (start 145.901 82.219) (end 145.901 88.580314) (width 0.2) (layer "F.Cu") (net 5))
 (segment (start 144.5 81.08) (end 144.5 88) (width 0.2) (layer "F.Cu") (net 12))
 (segment (start 150 75.58) (end 144.5 81.08) (width 0.2) (layer "F.Cu") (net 12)))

